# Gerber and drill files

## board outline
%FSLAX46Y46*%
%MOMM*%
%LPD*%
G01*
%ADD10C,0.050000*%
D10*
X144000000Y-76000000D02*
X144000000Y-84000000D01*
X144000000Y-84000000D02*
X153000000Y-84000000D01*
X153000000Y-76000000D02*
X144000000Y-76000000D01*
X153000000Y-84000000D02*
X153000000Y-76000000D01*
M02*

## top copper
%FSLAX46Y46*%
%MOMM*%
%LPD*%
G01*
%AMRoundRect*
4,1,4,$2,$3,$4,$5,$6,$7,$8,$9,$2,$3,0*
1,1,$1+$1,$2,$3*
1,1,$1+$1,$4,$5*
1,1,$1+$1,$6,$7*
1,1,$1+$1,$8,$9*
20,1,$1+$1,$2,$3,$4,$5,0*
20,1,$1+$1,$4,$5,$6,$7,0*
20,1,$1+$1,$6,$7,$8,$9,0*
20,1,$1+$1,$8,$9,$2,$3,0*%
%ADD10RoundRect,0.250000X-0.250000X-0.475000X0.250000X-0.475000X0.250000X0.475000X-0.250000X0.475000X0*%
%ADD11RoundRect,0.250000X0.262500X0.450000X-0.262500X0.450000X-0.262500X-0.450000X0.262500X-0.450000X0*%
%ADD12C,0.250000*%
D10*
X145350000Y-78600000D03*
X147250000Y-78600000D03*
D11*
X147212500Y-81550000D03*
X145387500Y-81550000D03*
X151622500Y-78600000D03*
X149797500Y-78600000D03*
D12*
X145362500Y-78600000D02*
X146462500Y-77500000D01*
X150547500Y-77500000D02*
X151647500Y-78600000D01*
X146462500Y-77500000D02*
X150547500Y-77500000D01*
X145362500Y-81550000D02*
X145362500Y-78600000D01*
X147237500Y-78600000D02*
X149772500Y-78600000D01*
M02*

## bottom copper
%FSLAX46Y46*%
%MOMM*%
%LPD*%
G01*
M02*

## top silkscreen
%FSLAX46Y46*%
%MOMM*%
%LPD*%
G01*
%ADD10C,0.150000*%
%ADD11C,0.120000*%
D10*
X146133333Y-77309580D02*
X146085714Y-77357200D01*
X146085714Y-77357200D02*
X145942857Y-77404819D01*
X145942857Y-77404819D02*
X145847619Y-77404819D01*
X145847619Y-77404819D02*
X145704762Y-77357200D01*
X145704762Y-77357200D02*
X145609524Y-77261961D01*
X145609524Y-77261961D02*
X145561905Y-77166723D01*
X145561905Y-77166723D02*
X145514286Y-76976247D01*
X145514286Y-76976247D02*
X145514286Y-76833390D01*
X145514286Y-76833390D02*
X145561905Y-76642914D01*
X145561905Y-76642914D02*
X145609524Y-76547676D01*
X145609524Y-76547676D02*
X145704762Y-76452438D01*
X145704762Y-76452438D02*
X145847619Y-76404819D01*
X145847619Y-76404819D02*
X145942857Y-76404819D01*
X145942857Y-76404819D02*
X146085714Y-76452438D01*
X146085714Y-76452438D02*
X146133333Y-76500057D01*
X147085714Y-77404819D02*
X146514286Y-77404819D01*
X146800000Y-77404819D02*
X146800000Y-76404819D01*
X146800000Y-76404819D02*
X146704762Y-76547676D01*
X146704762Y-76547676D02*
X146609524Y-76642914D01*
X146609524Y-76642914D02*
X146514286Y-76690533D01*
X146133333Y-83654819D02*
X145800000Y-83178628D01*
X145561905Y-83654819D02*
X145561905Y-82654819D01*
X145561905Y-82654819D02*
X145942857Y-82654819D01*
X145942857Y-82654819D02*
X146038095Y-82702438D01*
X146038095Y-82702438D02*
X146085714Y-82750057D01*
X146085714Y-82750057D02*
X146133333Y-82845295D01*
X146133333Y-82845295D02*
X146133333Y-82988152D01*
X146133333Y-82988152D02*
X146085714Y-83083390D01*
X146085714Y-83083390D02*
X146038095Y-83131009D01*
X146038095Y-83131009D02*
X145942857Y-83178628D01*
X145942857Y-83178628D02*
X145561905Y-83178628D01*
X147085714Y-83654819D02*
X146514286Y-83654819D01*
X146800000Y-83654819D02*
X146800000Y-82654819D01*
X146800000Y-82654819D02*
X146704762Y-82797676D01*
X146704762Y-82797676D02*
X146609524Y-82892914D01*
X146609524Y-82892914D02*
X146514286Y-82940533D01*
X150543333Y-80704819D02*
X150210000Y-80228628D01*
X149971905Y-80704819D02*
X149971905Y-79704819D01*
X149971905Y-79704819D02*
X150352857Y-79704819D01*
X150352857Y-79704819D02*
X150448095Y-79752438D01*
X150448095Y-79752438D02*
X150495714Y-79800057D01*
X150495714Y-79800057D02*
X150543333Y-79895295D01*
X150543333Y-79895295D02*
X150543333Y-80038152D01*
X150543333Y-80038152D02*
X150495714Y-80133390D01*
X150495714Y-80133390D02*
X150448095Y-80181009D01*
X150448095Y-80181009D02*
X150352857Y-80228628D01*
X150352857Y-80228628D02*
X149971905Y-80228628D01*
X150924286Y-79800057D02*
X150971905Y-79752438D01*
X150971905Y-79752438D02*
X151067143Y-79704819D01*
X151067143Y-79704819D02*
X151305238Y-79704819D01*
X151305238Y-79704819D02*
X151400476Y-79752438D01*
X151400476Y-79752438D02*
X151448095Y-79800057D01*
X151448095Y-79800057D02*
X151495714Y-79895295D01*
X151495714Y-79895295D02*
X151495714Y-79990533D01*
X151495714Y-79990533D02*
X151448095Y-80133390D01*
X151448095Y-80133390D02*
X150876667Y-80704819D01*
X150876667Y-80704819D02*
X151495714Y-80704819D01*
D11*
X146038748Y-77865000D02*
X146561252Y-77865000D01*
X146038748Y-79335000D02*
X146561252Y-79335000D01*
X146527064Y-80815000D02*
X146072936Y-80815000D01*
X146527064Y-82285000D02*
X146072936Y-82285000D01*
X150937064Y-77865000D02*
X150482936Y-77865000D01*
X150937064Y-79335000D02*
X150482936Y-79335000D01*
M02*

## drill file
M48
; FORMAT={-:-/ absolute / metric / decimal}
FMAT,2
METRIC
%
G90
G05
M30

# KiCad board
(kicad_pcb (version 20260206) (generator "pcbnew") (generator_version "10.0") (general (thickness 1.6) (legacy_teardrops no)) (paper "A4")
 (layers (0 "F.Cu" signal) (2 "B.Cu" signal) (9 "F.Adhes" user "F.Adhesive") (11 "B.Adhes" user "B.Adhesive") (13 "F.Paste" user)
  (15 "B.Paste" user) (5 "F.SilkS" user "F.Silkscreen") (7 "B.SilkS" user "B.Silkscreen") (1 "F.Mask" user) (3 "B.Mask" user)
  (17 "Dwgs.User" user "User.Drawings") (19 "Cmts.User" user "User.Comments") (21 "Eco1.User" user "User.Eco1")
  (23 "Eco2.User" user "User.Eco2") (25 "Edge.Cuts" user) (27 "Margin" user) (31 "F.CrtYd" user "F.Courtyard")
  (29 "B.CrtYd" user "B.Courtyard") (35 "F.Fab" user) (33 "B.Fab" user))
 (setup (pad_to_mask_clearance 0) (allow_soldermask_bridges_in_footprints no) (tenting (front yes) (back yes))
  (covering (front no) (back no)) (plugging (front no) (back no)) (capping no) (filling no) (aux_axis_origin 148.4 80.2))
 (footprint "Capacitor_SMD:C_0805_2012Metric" (layer "F.Cu") (at 146.3 78.6)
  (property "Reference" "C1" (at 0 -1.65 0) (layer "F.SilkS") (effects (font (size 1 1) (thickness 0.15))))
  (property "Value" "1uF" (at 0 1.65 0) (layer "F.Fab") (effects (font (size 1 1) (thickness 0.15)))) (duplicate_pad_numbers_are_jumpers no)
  (fp_line (start -0.261252 -0.735) (end 0.261252 -0.735) (stroke (width 0.12) (type solid)) (layer "F.SilkS"))
  (fp_line (start -0.261252 0.735) (end 0.261252 0.735) (stroke (width 0.12) (type solid)) (layer "F.SilkS"))
  (pad "1" smd roundrect (at -0.95 0) (size 1 1.45) (layers "F.Cu" "F.Mask" "F.Paste") (roundrect_rratio 0.25) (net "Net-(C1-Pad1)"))
  (pad "2" smd roundrect (at 0.95 0) (size 1 1.45) (layers "F.Cu" "F.Mask" "F.Paste") (roundrect_rratio 0.25) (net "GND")))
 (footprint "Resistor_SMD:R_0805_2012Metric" (layer "F.Cu") (at 146.3 81.55 180)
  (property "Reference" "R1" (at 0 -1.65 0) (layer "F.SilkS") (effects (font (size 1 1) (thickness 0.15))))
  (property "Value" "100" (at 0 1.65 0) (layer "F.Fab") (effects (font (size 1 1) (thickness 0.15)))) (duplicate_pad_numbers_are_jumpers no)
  (fp_line (start -0.227064 0.735) (end 0.227064 0.735) (stroke (width 0.12) (type solid)) (layer "F.SilkS"))
  (fp_line (start -0.227064 -0.735) (end 0.227064 -0.735) (stroke (width 0.12) (type solid)) (layer "F.SilkS"))
  (pad "1" smd roundrect (at -0.9125 0 180) (size 1.025 1.4) (layers "F.Cu" "F.Mask" "F.Paste") (roundrect_rratio 0.243902) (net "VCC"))
  (pad "2" smd roundrect (at 0.9125 0 180) (size 1.025 1.4) (layers "F.Cu" "F.Mask" "F.Paste") (roundrect_rratio 0.243902)
   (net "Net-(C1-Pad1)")))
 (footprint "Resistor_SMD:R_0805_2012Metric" (layer "F.Cu") (at 150.71 78.6 180)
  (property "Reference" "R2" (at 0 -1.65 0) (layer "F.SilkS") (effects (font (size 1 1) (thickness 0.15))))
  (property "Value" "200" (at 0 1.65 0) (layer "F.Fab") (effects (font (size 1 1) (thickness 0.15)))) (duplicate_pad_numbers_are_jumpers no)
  (fp_line (start -0.227064 0.735) (end 0.227064 0.735) (stroke (width 0.12) (type solid)) (layer "F.SilkS"))
  (fp_line (start -0.227064 -0.735) (end 0.227064 -0.735) (stroke (width 0.12) (type solid)) (layer "F.SilkS"))
  (pad "1" smd roundrect (at -0.9125 0 180) (size 1.025 1.4) (layers "F.Cu" "F.Mask" "F.Paste") (roundrect_rratio 0.243902)
   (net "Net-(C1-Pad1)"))
  (pad "2" smd roundrect (at 0.9125 0 180) (size 1.025 1.4) (layers "F.Cu" "F.Mask" "F.Paste") (roundrect_rratio 0.243902) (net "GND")))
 (gr_line (start 144 76) (end 144 84) (stroke (width 0.05) (type solid)) (layer "Edge.Cuts"))
 (gr_line (start 144 84) (end 153 84) (stroke (width 0.05) (type solid)) (layer "Edge.Cuts"))
 (gr_line (start 153 76) (end 144 76) (stroke (width 0.05) (type solid)) (layer "Edge.Cuts"))
 (gr_line (start 153 84) (end 153 76) (stroke (width 0.05) (type solid)) (layer "Edge.Cuts"))
 (segment (start 145.3625 78.6) (end 146.4625 77.5) (width 0.25) (layer "F.Cu") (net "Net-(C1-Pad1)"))
 (segment (start 150.5475 77.5) (end 151.6475 78.6) (width 0.25) (layer "F.Cu") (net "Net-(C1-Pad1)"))
 (segment (start 146.4625 77.5) (end 150.5475 77.5) (width 0.25) (layer "F.Cu") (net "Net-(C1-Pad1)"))
 (segment (start 145.3625 81.55) (end 145.3625 78.6) (width 0.25) (layer "F.Cu") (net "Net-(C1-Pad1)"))
 (segment (start 147.2375 78.6) (end 149.7725 78.6) (width 0.25) (layer "F.Cu") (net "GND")))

